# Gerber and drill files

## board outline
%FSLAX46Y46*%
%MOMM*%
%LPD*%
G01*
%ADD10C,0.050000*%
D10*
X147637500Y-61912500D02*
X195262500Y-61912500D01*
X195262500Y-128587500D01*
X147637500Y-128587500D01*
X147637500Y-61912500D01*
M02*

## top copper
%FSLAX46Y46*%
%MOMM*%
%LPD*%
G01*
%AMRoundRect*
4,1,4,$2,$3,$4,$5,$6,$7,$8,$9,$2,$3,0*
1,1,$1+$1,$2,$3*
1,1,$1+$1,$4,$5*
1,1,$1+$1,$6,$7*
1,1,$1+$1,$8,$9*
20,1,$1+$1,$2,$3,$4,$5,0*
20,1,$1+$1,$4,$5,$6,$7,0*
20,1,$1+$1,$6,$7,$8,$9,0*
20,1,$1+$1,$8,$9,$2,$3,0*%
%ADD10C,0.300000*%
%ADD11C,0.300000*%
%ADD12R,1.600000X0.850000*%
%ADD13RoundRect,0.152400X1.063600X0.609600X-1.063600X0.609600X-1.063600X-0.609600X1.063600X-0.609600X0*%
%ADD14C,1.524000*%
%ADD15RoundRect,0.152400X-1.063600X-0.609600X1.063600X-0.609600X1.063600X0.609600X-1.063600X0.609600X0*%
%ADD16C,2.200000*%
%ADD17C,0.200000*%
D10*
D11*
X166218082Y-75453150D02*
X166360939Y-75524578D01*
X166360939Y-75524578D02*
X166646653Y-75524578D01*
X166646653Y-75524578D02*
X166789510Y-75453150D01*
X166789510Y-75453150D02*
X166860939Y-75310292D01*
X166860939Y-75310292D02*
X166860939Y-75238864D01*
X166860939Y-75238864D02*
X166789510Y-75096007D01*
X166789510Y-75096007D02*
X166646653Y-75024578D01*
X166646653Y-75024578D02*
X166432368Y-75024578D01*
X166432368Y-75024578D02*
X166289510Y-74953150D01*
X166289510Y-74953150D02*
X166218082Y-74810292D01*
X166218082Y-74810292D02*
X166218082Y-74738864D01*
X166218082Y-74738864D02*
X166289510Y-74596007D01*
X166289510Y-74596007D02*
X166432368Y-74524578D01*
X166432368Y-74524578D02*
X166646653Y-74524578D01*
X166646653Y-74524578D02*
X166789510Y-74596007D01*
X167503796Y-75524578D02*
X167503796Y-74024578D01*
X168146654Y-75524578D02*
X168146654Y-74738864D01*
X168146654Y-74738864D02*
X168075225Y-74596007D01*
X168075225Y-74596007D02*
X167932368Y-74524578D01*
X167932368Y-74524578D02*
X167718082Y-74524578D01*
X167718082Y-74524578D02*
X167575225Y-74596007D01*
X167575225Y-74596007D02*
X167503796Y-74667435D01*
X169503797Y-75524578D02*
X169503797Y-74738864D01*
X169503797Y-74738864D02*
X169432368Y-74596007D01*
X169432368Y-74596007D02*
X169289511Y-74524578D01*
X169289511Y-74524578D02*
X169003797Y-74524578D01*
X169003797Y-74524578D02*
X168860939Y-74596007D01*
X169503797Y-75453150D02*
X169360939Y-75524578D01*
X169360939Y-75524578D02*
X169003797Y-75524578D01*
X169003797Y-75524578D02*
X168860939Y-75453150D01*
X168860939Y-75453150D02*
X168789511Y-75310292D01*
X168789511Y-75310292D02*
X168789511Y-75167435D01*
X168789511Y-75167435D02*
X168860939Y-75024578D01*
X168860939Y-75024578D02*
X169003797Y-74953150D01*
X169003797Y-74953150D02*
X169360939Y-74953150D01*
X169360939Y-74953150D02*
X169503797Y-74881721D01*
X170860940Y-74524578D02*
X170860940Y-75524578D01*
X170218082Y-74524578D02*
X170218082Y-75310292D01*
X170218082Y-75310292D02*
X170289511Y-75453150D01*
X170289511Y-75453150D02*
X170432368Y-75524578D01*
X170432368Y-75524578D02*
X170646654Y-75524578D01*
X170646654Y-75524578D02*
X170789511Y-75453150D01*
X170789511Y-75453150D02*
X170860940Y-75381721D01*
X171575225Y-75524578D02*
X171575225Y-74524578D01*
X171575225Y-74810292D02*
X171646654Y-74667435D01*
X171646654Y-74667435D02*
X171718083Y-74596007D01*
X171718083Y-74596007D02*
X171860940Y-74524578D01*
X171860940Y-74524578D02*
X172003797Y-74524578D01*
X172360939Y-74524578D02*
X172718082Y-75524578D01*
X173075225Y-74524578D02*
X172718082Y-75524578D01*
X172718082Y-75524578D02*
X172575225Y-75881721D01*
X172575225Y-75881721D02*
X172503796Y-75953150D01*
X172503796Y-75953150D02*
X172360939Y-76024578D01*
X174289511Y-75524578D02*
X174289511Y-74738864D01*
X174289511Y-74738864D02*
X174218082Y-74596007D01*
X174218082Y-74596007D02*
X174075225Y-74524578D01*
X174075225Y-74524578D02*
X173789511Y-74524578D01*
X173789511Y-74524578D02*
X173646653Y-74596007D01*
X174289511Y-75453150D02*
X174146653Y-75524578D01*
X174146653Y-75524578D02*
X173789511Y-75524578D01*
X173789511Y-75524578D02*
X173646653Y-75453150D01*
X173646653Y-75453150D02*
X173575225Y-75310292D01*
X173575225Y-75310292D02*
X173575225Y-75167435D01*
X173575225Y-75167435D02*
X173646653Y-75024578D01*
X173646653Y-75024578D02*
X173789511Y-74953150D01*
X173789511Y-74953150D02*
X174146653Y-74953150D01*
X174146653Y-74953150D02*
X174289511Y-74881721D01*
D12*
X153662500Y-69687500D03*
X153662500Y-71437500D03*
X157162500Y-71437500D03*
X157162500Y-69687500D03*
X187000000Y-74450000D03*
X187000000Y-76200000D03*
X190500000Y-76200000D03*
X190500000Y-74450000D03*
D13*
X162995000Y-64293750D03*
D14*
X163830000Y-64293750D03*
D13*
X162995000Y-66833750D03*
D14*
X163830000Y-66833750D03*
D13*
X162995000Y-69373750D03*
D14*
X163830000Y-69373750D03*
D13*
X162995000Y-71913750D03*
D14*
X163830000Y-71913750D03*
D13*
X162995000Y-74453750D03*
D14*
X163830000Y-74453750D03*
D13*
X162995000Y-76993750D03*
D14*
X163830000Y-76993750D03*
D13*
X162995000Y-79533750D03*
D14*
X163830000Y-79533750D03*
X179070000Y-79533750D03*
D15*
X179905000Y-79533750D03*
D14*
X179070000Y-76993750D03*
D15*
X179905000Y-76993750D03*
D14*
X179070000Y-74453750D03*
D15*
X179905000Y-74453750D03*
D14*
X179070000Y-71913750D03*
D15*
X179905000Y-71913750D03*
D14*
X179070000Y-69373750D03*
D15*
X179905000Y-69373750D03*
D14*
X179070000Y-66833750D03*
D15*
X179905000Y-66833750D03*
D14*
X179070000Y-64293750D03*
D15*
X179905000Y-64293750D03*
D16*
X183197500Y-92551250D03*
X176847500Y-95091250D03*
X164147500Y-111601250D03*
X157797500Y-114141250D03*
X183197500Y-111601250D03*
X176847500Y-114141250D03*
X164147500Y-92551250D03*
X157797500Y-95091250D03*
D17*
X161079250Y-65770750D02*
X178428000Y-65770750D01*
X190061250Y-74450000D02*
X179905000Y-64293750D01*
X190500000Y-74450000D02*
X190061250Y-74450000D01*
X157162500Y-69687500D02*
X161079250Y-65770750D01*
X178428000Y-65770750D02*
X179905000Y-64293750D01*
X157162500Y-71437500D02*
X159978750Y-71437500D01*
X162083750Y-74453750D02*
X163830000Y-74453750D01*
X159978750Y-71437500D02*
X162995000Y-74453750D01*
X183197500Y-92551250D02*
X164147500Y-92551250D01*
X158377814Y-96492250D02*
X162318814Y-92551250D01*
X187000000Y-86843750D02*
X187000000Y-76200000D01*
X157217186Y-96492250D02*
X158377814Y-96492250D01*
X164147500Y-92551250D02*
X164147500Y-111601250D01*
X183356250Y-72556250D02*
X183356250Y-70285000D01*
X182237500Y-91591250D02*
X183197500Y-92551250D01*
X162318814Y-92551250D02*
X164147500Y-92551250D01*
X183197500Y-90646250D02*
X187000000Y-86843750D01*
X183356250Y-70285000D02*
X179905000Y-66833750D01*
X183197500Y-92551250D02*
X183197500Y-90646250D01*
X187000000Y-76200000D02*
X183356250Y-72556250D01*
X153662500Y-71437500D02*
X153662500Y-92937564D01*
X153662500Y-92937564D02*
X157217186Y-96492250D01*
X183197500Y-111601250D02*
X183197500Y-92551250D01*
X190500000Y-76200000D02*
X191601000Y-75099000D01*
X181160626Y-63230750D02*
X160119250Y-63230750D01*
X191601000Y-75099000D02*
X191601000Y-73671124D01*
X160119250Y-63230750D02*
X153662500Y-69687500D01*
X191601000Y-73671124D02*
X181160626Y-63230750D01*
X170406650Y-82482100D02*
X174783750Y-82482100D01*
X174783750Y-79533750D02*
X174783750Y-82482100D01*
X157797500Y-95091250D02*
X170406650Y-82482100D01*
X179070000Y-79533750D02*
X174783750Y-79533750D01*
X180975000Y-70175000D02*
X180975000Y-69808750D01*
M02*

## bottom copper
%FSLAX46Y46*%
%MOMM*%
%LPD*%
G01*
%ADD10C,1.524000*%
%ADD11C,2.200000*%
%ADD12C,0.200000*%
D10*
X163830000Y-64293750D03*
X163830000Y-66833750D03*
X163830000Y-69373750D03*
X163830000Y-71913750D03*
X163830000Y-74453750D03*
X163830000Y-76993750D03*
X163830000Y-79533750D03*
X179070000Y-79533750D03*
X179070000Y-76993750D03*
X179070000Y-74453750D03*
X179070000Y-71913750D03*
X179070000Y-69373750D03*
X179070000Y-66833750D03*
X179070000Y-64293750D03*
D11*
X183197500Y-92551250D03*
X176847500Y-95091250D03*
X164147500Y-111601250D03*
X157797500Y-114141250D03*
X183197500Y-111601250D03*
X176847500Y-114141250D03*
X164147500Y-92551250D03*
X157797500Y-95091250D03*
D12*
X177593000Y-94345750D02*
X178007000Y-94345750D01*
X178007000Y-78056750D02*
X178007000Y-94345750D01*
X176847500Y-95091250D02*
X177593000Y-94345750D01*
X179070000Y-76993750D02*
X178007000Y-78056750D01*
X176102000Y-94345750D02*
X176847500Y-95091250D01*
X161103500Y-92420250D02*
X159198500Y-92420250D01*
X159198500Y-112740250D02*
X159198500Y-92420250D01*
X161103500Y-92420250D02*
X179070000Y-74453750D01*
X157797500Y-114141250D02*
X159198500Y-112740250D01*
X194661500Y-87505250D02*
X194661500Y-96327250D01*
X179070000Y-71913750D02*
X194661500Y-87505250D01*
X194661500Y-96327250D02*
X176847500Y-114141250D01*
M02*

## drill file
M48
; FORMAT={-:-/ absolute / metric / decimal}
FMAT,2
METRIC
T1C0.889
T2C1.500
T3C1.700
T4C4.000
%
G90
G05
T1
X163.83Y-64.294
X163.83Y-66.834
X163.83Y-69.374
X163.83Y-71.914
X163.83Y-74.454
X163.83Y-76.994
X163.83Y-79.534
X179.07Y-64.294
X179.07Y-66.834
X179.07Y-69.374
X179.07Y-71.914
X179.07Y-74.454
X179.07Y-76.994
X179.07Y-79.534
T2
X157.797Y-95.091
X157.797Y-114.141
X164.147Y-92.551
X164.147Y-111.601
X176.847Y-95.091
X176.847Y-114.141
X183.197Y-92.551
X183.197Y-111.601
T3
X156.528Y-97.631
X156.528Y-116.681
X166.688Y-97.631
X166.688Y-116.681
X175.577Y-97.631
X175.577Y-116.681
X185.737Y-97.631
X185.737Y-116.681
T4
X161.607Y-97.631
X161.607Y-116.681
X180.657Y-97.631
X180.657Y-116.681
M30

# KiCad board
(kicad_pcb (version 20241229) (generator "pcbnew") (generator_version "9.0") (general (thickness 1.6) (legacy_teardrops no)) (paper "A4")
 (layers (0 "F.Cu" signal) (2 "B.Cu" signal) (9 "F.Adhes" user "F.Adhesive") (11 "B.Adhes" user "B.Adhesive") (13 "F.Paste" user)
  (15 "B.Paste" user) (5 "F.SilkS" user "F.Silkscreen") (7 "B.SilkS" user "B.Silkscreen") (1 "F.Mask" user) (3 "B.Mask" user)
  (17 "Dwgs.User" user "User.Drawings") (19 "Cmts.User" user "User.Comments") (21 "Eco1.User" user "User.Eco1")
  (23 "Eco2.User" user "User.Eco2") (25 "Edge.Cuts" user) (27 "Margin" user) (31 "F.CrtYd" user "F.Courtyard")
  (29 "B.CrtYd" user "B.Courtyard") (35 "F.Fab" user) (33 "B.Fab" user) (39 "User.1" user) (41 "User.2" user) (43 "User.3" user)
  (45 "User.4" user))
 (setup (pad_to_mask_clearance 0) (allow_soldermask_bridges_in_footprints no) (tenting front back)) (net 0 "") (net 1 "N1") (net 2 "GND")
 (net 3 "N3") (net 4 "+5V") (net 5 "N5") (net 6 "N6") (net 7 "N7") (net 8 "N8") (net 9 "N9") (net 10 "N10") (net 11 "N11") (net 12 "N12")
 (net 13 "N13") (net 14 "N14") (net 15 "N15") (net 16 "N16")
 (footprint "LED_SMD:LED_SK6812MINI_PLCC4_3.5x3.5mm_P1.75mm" (layer "F.Cu") (at 155.4125 70.5625)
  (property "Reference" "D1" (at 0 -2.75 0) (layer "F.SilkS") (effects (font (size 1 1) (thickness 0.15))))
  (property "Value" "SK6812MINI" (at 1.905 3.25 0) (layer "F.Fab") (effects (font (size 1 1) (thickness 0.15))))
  (pad "1" smd rect (at -1.75 -0.875) (size 1.6 0.85) (layers "F.Cu" "F.Mask" "F.Paste") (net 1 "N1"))
  (pad "2" smd rect (at -1.75 0.875) (size 1.6 0.85) (layers "F.Cu" "F.Mask" "F.Paste") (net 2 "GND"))
  (pad "3" smd rect (at 1.75 0.875) (size 1.6 0.85) (layers "F.Cu" "F.Mask" "F.Paste") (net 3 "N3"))
  (pad "4" smd rect (at 1.75 -0.875) (size 1.6 0.85) (layers "F.Cu" "F.Mask" "F.Paste") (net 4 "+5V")))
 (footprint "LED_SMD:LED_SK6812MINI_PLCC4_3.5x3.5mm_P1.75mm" (layer "F.Cu") (at 188.75 75.325)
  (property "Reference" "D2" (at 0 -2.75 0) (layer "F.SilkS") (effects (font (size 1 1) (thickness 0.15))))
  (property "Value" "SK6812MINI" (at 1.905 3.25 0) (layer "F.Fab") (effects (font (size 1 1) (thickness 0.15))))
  (pad "1" smd rect (at -1.75 -0.875) (size 1.6 0.85) (layers "F.Cu" "F.Mask" "F.Paste") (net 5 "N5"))
  (pad "2" smd rect (at -1.75 0.875) (size 1.6 0.85) (layers "F.Cu" "F.Mask" "F.Paste") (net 2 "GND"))
  (pad "3" smd rect (at 1.75 0.875) (size 1.6 0.85) (layers "F.Cu" "F.Mask" "F.Paste") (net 1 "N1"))
  (pad "4" smd rect (at 1.75 -0.875) (size 1.6 0.85) (layers "F.Cu" "F.Mask" "F.Paste") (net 4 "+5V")))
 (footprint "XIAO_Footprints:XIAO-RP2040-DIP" (layer "F.Cu") (at 171.45 71.91375)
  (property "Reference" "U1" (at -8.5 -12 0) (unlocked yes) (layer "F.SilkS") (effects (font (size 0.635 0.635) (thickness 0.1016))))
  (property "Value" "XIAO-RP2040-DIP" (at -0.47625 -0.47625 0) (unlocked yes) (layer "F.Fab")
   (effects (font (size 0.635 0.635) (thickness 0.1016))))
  (pad "1" smd roundrect (at -8.455 -7.62 180) (size 2.432 1.524) (layers "F.Cu" "F.Mask") (roundrect_rratio 0.1) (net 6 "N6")
   (thermal_bridge_angle 45))
  (pad "1" thru_hole circle (at -7.62 -7.62 180) (size 1.524 1.524) (drill 0.889) (layers "*.Cu" "*.Mask") (remove_unused_layers no)
   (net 6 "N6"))
  (pad "2" smd roundrect (at -8.455 -5.08 180) (size 2.432 1.524) (layers "F.Cu" "F.Mask") (roundrect_rratio 0.1) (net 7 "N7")
   (thermal_bridge_angle 45))
  (pad "2" thru_hole circle (at -7.62 -5.08 180) (size 1.524 1.524) (drill 0.889) (layers "*.Cu" "*.Mask") (remove_unused_layers no)
   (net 7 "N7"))
  (pad "3" smd roundrect (at -8.455 -2.54 180) (size 2.432 1.524) (layers "F.Cu" "F.Mask") (roundrect_rratio 0.1) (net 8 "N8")
   (thermal_bridge_angle 45))
  (pad "3" thru_hole circle (at -7.62 -2.54 180) (size 1.524 1.524) (drill 0.889) (layers "*.Cu" "*.Mask") (remove_unused_layers no)
   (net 8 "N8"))
  (pad "4" smd roundrect (at -8.455 0 180) (size 2.432 1.524) (layers "F.Cu" "F.Mask") (roundrect_rratio 0.1) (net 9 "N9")
   (thermal_bridge_angle 45))
  (pad "4" thru_hole circle (at -7.62 0 180) (size 1.524 1.524) (drill 0.889) (layers "*.Cu" "*.Mask") (remove_unused_layers no)
   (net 9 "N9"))
  (pad "5" smd roundrect (at -8.455 2.54 180) (size 2.432 1.524) (layers "F.Cu" "F.Mask") (roundrect_rratio 0.1) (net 3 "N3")
   (thermal_bridge_angle 45))
  (pad "5" thru_hole circle (at -7.62 2.54 180) (size 1.524 1.524) (drill 0.889) (layers "*.Cu" "*.Mask") (remove_unused_layers no)
   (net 3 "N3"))
  (pad "6" smd roundrect (at -8.455 5.08 180) (size 2.432 1.524) (layers "F.Cu" "F.Mask") (roundrect_rratio 0.1) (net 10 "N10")
   (thermal_bridge_angle 45))
  (pad "6" thru_hole circle (at -7.62 5.08 180) (size 1.524 1.524) (drill 0.889) (layers "*.Cu" "*.Mask") (remove_unused_layers no)
   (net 10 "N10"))
  (pad "7" smd roundrect (at -8.455 7.62 180) (size 2.432 1.524) (layers "F.Cu" "F.Mask") (roundrect_rratio 0.1) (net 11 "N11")
   (thermal_bridge_angle 45))
  (pad "7" thru_hole circle (at -7.62 7.62 180) (size 1.524 1.524) (drill 0.889) (layers "*.Cu" "*.Mask") (remove_unused_layers no)
   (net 11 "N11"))
  (pad "8" thru_hole circle (at 7.62 7.62) (size 1.524 1.524) (drill 0.889) (layers "*.Cu" "*.Mask") (remove_unused_layers no)
   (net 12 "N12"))
  (pad "8" smd roundrect (at 8.455 7.62) (size 2.432 1.524) (layers "F.Cu" "F.Mask") (roundrect_rratio 0.1) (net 12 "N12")
   (thermal_bridge_angle 45))
  (pad "9" thru_hole circle (at 7.62 5.08) (size 1.524 1.524) (drill 0.889) (layers "*.Cu" "*.Mask") (remove_unused_layers no)
   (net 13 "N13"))
  (pad "9" smd roundrect (at 8.455 5.08) (size 2.432 1.524) (layers "F.Cu" "F.Mask") (roundrect_rratio 0.1) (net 13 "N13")
   (thermal_bridge_angle 45))
  (pad "10" thru_hole circle (at 7.62 2.54) (size 1.524 1.524) (drill 0.889) (layers "*.Cu" "*.Mask") (remove_unused_layers no)
   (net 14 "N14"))
  (pad "10" smd roundrect (at 8.455 2.54) (size 2.432 1.524) (layers "F.Cu" "F.Mask") (roundrect_rratio 0.1) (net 14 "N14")
   (thermal_bridge_angle 45))
  (pad "11" thru_hole circle (at 7.62 0) (size 1.524 1.524) (drill 0.889) (layers "*.Cu" "*.Mask") (remove_unused_layers no) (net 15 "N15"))
  (pad "11" smd roundrect (at 8.455 0) (size 2.432 1.524) (layers "F.Cu" "F.Mask") (roundrect_rratio 0.1) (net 15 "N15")
   (thermal_bridge_angle 45))
  (pad "12" thru_hole circle (at 7.62 -2.54) (size 1.524 1.524) (drill 0.889) (layers "*.Cu" "*.Mask") (remove_unused_layers no)
   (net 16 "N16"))
  (pad "12" smd roundrect (at 8.455 -2.54) (size 2.432 1.524) (layers "F.Cu" "F.Mask") (roundrect_rratio 0.1) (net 16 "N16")
   (thermal_bridge_angle 45))
  (pad "13" thru_hole circle (at 7.62 -5.08) (size 1.524 1.524) (drill 0.889) (layers "*.Cu" "*.Mask") (remove_unused_layers no)
   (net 2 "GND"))
  (pad "13" smd roundrect (at 8.455 -5.08) (size 2.432 1.524) (layers "F.Cu" "F.Mask") (roundrect_rratio 0.1) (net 2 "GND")
   (thermal_bridge_angle 45))
  (pad "14" thru_hole circle (at 7.62 -7.62) (size 1.524 1.524) (drill 0.889) (layers "*.Cu" "*.Mask") (remove_unused_layers no)
   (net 4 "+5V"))
  (pad "14" smd roundrect (at 8.455 -7.62) (size 2.432 1.524) (layers "F.Cu" "F.Mask") (roundrect_rratio 0.1) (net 4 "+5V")
   (thermal_bridge_angle 45)))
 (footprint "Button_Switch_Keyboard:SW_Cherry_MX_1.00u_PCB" (layer "F.Cu") (at 183.1975 92.55125)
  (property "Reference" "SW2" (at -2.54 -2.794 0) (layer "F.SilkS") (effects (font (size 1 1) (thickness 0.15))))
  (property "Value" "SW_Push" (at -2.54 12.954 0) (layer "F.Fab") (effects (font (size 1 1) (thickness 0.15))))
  (pad "" np_thru_hole circle (at -7.62 5.08) (size 1.7 1.7) (drill 1.7) (layers "*.Cu" "*.Mask"))
  (pad "" np_thru_hole circle (at -2.54 5.08) (size 4 4) (drill 4) (layers "*.Cu" "*.Mask"))
  (pad "" np_thru_hole circle (at 2.54 5.08) (size 1.7 1.7) (drill 1.7) (layers "*.Cu" "*.Mask"))
  (pad "1" thru_hole circle (at 0 0) (size 2.2 2.2) (drill 1.5) (layers "*.Cu" "*.Mask") (remove_unused_layers no) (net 2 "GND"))
  (pad "2" thru_hole circle (at -6.35 2.54) (size 2.2 2.2) (drill 1.5) (layers "*.Cu" "*.Mask") (remove_unused_layers no) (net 13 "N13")))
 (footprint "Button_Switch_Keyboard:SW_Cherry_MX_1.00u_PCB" (layer "F.Cu") (at 164.1475 111.60125)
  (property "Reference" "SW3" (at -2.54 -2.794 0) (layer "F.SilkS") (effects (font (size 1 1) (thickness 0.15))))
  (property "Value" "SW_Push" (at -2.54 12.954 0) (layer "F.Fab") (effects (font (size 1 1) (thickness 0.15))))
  (pad "" np_thru_hole circle (at -7.62 5.08) (size 1.7 1.7) (drill 1.7) (layers "*.Cu" "*.Mask"))
  (pad "" np_thru_hole circle (at -2.54 5.08) (size 4 4) (drill 4) (layers "*.Cu" "*.Mask"))
  (pad "" np_thru_hole circle (at 2.54 5.08) (size 1.7 1.7) (drill 1.7) (layers "*.Cu" "*.Mask"))
  (pad "1" thru_hole circle (at 0 0) (size 2.2 2.2) (drill 1.5) (layers "*.Cu" "*.Mask") (remove_unused_layers no) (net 2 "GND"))
  (pad "2" thru_hole circle (at -6.35 2.54) (size 2.2 2.2) (drill 1.5) (layers "*.Cu" "*.Mask") (remove_unused_layers no) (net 14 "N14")))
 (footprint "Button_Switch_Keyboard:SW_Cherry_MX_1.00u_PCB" (layer "F.Cu") (at 183.1975 111.60125)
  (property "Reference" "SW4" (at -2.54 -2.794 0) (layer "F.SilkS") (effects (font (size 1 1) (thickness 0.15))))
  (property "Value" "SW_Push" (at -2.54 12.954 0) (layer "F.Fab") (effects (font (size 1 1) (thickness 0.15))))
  (pad "" np_thru_hole circle (at -7.62 5.08) (size 1.7 1.7) (drill 1.7) (layers "*.Cu" "*.Mask"))
  (pad "" np_thru_hole circle (at -2.54 5.08) (size 4 4) (drill 4) (layers "*.Cu" "*.Mask"))
  (pad "" np_thru_hole circle (at 2.54 5.08) (size 1.7 1.7) (drill 1.7) (layers "*.Cu" "*.Mask"))
  (pad "1" thru_hole circle (at 0 0) (size 2.2 2.2) (drill 1.5) (layers "*.Cu" "*.Mask") (remove_unused_layers no) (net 2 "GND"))
  (pad "2" thru_hole circle (at -6.35 2.54) (size 2.2 2.2) (drill 1.5) (layers "*.Cu" "*.Mask") (remove_unused_layers no) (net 15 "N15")))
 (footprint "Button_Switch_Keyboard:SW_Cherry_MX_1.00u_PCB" (layer "F.Cu") (at 164.1475 92.55125)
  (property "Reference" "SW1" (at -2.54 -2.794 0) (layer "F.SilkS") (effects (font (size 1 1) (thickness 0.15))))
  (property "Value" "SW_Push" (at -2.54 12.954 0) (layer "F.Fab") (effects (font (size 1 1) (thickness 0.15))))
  (pad "" np_thru_hole circle (at -7.62 5.08) (size 1.7 1.7) (drill 1.7) (layers "*.Cu" "*.Mask"))
  (pad "" np_thru_hole circle (at -2.54 5.08) (size 4 4) (drill 4) (layers "*.Cu" "*.Mask"))
  (pad "" np_thru_hole circle (at 2.54 5.08) (size 1.7 1.7) (drill 1.7) (layers "*.Cu" "*.Mask"))
  (pad "1" thru_hole circle (at 0 0) (size 2.2 2.2) (drill 1.5) (layers "*.Cu" "*.Mask") (remove_unused_layers no) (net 2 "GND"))
  (pad "2" thru_hole circle (at -6.35 2.54) (size 2.2 2.2) (drill 1.5) (layers "*.Cu" "*.Mask") (remove_unused_layers no) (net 12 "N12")))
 (gr_rect (start 147.6375 61.9125) (end 195.2625 128.5875) (stroke (width 0.05) (type default)) (fill no) (layer "Edge.Cuts"))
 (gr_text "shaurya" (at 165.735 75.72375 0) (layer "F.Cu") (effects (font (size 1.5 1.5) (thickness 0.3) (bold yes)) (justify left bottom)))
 (segment (start 161.07925 65.77075) (end 178.428 65.77075) (width 0.2) (layer "F.Cu") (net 4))
 (segment (start 190.06125 74.45) (end 179.905 64.29375) (width 0.2) (layer "F.Cu") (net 4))
 (segment (start 190.5 74.45) (end 190.06125 74.45) (width 0.2) (layer "F.Cu") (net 4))
 (segment (start 157.1625 69.6875) (end 161.07925 65.77075) (width 0.2) (layer "F.Cu") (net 4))
 (segment (start 178.428 65.77075) (end 179.905 64.29375) (width 0.2) (layer "F.Cu") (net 4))
 (segment (start 157.1625 71.4375) (end 159.97875 71.4375) (width 0.2) (layer "F.Cu") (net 3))
 (segment (start 162.08375 74.45375) (end 163.83 74.45375) (width 0.2) (layer "F.Cu") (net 3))
 (segment (start 159.97875 71.4375) (end 162.995 74.45375) (width 0.2) (layer "F.Cu") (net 3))
 (segment (start 183.1975 92.55125) (end 164.1475 92.55125) (width 0.2) (layer "F.Cu") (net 2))
 (segment (start 158.377814 96.49225) (end 162.318814 92.55125) (width 0.2) (layer "F.Cu") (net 2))
 (segment (start 187 86.84375) (end 187 76.2) (width 0.2) (layer "F.Cu") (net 2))
 (segment (start 157.217186 96.49225) (end 158.377814 96.49225) (width 0.2) (layer "F.Cu") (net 2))
 (segment (start 164.1475 92.55125) (end 164.1475 111.60125) (width 0.2) (layer "F.Cu") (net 2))
 (segment (start 183.35625 72.55625) (end 183.35625 70.285) (width 0.2) (layer "F.Cu") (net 2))
 (segment (start 182.2375 91.59125) (end 183.1975 92.55125) (width 0.2) (layer "F.Cu") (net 2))
 (segment (start 162.318814 92.55125) (end 164.1475 92.55125) (width 0.2) (layer "F.Cu") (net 2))
 (segment (start 183.1975 90.64625) (end 187 86.84375) (width 0.2) (layer "F.Cu") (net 2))
 (segment (start 183.35625 70.285) (end 179.905 66.83375) (width 0.2) (layer "F.Cu") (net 2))
 (segment (start 183.1975 92.55125) (end 183.1975 90.64625) (width 0.2) (layer "F.Cu") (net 2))
 (segment (start 187 76.2) (end 183.35625 72.55625) (width 0.2) (layer "F.Cu") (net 2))
 (segment (start 153.6625 71.4375) (end 153.6625 92.937564) (width 0.2) (layer "F.Cu") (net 2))
 (segment (start 153.6625 92.937564) (end 157.217186 96.49225) (width 0.2) (layer "F.Cu") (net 2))
 (segment (start 183.1975 111.60125) (end 183.1975 92.55125) (width 0.2) (layer "F.Cu") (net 2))
 (segment (start 190.5 76.2) (end 191.601 75.099) (width 0.2) (layer "F.Cu") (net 1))
 (segment (start 181.160626 63.23075) (end 160.11925 63.23075) (width 0.2) (layer "F.Cu") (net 1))
 (segment (start 191.601 75.099) (end 191.601 73.671124) (width 0.2) (layer "F.Cu") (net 1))
 (segment (start 160.11925 63.23075) (end 153.6625 69.6875) (width 0.2) (layer "F.Cu") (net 1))
 (segment (start 191.601 73.671124) (end 181.160626 63.23075) (width 0.2) (layer "F.Cu") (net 1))
 (segment (start 170.40665 82.4821) (end 174.78375 82.4821) (width 0.2) (layer "F.Cu") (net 12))
 (segment (start 174.78375 79.53375) (end 174.78375 82.4821) (width 0.2) (layer "F.Cu") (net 12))
 (segment (start 157.7975 95.09125) (end 170.40665 82.4821) (width 0.2) (layer "F.Cu") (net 12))
 (segment (start 179.07 79.53375) (end 174.78375 79.53375) (width 0.2) (layer "F.Cu") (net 12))
 (segment (start 177.593 94.34575) (end 178.007 94.34575) (width 0.2) (layer "B.Cu") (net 13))
 (segment (start 178.007 78.05675) (end 178.007 94.34575) (width 0.2) (layer "B.Cu") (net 13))
 (segment (start 176.8475 95.09125) (end 177.593 94.34575) (width 0.2) (layer "B.Cu") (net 13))
 (segment (start 179.07 76.99375) (end 178.007 78.05675) (width 0.2) (layer "B.Cu") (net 13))
 (segment (start 176.102 94.34575) (end 176.8475 95.09125) (width 0.2) (layer "B.Cu") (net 13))
 (segment (start 161.1035 92.42025) (end 159.1985 92.42025) (width 0.2) (layer "B.Cu") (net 14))
 (segment (start 159.1985 112.74025) (end 159.1985 92.42025) (width 0.2) (layer "B.Cu") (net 14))
 (segment (start 161.1035 92.42025) (end 179.07 74.45375) (width 0.2) (layer "B.Cu") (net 14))
 (segment (start 157.7975 114.14125) (end 159.1985 112.74025) (width 0.2) (layer "B.Cu") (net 14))
 (segment (start 194.6615 87.50525) (end 194.6615 96.32725) (width 0.2) (layer "B.Cu") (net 15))
 (segment (start 179.07 71.91375) (end 194.6615 87.50525) (width 0.2) (layer "B.Cu") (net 15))
 (segment (start 194.6615 96.32725) (end 176.8475 114.14125) (width 0.2) (layer "B.Cu") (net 15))
 (segment (start 180.975 70.175) (end 180.975 69.80875) (width 0.2) (layer "F.Cu") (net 16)))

